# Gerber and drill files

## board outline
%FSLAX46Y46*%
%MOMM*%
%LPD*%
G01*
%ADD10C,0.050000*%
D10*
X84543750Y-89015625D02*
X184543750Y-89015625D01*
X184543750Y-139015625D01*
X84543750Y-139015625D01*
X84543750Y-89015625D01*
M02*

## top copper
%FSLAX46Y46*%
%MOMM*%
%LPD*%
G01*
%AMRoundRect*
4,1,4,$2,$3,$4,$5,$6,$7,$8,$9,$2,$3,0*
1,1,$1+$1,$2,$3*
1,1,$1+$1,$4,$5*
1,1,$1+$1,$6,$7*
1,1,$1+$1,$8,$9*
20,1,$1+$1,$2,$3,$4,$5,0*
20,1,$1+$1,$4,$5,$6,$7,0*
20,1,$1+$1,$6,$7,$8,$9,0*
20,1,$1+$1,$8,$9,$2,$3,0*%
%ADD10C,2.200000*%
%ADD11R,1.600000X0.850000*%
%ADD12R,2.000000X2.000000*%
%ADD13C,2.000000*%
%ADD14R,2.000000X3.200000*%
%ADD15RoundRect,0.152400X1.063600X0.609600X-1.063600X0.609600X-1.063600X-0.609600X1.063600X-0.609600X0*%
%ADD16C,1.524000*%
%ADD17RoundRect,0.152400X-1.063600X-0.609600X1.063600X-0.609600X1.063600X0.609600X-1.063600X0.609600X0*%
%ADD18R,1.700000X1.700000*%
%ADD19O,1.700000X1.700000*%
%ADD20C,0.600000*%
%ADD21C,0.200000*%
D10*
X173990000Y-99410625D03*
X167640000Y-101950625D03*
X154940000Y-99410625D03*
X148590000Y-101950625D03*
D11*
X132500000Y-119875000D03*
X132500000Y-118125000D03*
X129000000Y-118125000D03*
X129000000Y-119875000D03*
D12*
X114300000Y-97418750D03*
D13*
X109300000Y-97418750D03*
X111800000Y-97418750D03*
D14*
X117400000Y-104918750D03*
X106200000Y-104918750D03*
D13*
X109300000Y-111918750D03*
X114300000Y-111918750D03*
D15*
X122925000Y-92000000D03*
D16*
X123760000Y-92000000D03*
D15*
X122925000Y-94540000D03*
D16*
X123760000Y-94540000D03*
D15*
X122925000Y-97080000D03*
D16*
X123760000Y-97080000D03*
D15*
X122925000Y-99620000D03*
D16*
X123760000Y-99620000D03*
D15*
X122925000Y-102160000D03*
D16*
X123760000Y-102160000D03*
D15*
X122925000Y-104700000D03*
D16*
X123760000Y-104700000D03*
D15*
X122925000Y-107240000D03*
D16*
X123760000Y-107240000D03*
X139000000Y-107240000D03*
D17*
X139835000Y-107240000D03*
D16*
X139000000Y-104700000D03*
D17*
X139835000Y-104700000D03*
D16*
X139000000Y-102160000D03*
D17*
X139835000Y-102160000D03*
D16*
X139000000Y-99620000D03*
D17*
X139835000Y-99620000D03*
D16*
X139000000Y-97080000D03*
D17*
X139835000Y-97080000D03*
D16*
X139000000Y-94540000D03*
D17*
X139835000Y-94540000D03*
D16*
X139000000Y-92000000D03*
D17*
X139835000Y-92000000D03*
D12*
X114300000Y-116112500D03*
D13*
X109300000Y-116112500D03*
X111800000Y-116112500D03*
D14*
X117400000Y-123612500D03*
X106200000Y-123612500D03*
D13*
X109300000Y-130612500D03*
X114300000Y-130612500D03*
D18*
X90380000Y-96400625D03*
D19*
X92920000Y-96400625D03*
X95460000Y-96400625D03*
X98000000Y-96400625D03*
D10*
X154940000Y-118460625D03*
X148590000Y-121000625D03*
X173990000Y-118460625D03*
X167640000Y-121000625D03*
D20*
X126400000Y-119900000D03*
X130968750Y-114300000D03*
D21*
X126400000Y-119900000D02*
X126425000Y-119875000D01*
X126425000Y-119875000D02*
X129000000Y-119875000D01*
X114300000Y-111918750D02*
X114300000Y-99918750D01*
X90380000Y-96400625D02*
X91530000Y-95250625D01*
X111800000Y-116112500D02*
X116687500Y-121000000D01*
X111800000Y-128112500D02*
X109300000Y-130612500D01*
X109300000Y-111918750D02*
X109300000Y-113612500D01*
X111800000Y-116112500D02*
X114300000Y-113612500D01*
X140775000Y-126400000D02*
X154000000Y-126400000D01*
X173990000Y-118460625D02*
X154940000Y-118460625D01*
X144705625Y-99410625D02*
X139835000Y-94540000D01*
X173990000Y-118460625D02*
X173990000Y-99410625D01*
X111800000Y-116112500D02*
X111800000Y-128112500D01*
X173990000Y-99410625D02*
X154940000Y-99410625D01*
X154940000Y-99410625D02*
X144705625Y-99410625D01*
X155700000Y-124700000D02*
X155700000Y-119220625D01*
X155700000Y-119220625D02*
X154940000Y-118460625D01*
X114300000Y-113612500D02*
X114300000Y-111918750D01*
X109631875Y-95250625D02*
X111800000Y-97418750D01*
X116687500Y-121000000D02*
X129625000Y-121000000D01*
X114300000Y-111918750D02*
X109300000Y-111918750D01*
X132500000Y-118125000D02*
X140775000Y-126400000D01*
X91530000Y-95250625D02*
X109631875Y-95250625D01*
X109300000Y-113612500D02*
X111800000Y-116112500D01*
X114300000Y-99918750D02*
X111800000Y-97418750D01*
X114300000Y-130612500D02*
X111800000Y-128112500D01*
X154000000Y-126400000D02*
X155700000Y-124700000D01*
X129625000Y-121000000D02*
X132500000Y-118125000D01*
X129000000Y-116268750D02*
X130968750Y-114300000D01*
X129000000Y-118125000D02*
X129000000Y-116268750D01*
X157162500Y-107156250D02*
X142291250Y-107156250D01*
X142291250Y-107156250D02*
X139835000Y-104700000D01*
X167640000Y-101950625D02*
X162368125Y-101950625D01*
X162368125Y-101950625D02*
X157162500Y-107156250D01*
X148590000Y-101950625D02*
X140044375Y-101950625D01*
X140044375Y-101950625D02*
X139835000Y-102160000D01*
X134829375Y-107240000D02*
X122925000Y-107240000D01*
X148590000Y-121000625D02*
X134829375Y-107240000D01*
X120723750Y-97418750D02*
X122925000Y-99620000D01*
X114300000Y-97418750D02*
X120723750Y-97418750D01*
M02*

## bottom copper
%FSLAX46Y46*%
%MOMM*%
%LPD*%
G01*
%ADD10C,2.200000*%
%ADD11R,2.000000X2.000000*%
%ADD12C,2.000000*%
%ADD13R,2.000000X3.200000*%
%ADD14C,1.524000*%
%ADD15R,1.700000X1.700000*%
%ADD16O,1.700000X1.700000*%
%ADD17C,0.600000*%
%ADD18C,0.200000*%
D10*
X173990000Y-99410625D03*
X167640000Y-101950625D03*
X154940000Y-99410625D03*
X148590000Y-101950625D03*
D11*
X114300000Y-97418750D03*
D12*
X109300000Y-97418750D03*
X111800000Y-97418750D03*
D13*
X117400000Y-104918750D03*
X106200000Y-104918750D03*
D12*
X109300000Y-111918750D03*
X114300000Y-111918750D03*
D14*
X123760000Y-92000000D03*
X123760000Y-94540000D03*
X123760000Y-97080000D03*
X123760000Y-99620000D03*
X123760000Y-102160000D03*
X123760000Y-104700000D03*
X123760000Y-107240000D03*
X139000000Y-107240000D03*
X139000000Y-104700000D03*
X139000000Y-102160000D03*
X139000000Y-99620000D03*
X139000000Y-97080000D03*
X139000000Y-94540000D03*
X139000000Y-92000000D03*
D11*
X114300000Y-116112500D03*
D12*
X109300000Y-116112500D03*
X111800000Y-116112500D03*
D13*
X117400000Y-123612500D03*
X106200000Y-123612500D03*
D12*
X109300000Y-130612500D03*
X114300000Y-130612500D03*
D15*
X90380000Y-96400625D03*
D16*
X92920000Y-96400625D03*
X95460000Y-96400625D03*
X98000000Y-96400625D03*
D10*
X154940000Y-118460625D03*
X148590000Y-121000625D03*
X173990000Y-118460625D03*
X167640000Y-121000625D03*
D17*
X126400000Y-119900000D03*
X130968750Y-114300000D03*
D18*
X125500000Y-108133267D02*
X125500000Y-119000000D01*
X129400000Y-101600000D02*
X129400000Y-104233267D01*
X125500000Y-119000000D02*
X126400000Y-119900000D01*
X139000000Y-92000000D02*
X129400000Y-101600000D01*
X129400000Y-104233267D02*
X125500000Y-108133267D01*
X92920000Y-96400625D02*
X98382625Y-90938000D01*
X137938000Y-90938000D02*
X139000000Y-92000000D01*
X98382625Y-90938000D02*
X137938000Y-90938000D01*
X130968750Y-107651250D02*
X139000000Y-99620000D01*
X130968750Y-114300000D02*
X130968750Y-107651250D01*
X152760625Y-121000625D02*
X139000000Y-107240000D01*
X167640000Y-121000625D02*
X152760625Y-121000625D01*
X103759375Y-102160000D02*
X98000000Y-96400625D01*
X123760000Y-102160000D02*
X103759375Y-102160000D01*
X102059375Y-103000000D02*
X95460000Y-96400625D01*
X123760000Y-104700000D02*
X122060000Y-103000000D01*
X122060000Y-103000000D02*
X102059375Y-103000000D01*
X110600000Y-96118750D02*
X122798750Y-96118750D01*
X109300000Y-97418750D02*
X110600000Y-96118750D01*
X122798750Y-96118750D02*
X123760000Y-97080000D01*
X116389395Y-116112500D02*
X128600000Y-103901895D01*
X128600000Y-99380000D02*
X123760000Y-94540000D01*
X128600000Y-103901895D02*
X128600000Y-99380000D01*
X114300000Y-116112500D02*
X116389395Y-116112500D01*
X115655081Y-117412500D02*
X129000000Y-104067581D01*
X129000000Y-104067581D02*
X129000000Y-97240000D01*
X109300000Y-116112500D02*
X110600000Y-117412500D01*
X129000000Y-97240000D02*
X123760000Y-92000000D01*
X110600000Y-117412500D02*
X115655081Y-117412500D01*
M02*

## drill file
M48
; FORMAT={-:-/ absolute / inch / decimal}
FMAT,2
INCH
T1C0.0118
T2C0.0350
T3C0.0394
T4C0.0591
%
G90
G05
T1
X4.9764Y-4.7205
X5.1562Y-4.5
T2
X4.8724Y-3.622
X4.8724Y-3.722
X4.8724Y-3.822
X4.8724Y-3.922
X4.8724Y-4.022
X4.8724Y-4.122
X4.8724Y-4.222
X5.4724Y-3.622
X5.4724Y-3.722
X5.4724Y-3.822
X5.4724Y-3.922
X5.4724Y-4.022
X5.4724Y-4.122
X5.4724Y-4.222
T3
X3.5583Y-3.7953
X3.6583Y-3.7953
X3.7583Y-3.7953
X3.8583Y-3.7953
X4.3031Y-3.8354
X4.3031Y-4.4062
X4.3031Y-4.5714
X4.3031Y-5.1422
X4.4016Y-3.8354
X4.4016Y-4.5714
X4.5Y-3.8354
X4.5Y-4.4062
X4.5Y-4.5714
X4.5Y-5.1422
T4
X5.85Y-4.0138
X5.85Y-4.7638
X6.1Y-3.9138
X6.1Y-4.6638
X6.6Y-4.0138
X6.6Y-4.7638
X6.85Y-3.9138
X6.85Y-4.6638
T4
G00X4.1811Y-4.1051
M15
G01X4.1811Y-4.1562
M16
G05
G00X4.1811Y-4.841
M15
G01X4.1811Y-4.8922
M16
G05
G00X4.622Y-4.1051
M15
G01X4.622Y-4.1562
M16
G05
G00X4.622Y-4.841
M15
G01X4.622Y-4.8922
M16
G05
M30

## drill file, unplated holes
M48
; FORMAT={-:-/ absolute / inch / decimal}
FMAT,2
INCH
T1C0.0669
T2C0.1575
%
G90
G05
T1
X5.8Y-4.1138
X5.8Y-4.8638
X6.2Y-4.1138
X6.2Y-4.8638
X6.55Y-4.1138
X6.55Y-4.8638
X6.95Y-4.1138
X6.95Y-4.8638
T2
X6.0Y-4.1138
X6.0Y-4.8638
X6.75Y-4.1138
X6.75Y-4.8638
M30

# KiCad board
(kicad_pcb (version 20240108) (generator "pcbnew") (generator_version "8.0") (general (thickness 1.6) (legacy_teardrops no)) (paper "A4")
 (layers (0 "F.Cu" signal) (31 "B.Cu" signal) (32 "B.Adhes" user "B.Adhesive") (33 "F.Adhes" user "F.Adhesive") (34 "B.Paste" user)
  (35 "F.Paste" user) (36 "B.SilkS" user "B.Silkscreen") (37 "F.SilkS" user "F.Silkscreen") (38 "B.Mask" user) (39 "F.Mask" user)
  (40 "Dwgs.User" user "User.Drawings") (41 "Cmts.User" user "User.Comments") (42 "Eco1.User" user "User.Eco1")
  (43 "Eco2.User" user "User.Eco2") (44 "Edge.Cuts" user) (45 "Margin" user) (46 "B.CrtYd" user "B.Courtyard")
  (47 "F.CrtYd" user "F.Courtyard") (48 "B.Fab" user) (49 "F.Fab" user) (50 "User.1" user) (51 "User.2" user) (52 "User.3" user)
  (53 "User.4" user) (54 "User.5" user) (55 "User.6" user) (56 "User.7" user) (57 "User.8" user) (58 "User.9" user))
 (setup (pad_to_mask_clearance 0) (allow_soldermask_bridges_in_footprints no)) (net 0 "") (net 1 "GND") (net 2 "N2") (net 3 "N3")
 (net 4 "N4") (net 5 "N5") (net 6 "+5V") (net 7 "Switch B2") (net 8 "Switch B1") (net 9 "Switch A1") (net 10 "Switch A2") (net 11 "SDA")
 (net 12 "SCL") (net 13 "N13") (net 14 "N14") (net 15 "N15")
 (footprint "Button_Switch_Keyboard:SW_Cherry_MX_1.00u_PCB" (layer "F.Cu") (at 173.99 99.410625)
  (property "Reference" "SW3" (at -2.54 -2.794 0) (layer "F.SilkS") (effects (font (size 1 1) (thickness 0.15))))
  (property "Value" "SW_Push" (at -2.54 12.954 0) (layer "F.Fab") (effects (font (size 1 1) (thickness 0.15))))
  (pad "" np_thru_hole circle (at -7.62 5.08) (size 1.7 1.7) (drill 1.7) (layers "*.Cu" "*.Mask"))
  (pad "" np_thru_hole circle (at -2.54 5.08) (size 4 4) (drill 4) (layers "*.Cu" "*.Mask"))
  (pad "" np_thru_hole circle (at 2.54 5.08) (size 1.7 1.7) (drill 1.7) (layers "*.Cu" "*.Mask"))
  (pad "1" thru_hole circle (at 0 0) (size 2.2 2.2) (drill 1.5) (layers "*.Cu" "*.Mask") (remove_unused_layers no) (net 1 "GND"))
  (pad "2" thru_hole circle (at -6.35 2.54) (size 2.2 2.2) (drill 1.5) (layers "*.Cu" "*.Mask") (remove_unused_layers no) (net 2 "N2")))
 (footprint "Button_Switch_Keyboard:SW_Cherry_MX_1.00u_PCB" (layer "F.Cu") (at 154.94 99.410625)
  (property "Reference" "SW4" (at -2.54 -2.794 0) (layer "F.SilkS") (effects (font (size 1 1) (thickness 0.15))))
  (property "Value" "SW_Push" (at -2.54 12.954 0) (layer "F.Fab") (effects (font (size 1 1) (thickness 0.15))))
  (pad "" np_thru_hole circle (at -7.62 5.08) (size 1.7 1.7) (drill 1.7) (layers "*.Cu" "*.Mask"))
  (pad "" np_thru_hole circle (at -2.54 5.08) (size 4 4) (drill 4) (layers "*.Cu" "*.Mask"))
  (pad "" np_thru_hole circle (at 2.54 5.08) (size 1.7 1.7) (drill 1.7) (layers "*.Cu" "*.Mask"))
  (pad "1" thru_hole circle (at 0 0) (size 2.2 2.2) (drill 1.5) (layers "*.Cu" "*.Mask") (remove_unused_layers no) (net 1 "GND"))
  (pad "2" thru_hole circle (at -6.35 2.54) (size 2.2 2.2) (drill 1.5) (layers "*.Cu" "*.Mask") (remove_unused_layers no) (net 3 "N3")))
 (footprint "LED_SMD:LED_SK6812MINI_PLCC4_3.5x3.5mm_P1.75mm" (layer "F.Cu") (at 130.75 119 180)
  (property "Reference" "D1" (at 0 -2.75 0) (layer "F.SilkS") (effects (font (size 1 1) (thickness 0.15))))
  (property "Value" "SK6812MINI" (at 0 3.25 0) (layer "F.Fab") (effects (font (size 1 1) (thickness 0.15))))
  (pad "1" smd rect (at -1.75 -0.875 180) (size 1.6 0.85) (layers "F.Cu" "F.Paste" "F.Mask") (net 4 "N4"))
  (pad "2" smd rect (at -1.75 0.875 180) (size 1.6 0.85) (layers "F.Cu" "F.Paste" "F.Mask") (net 1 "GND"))
  (pad "3" smd rect (at 1.75 0.875 180) (size 1.6 0.85) (layers "F.Cu" "F.Paste" "F.Mask") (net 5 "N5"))
  (pad "4" smd rect (at 1.75 -0.875 180) (size 1.6 0.85) (layers "F.Cu" "F.Paste" "F.Mask") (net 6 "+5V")))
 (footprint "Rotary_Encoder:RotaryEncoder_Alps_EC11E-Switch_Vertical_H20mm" (layer "F.Cu") (at 114.3 97.41875 -90)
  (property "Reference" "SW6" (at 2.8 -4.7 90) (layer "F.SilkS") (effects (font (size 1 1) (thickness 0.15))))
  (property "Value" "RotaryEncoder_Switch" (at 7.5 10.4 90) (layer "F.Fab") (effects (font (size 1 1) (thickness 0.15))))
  (pad "A" thru_hole rect (at 0 0 270) (size 2 2) (drill 1) (layers "*.Cu" "*.Mask") (remove_unused_layers no) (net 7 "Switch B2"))
  (pad "B" thru_hole circle (at 0 5 270) (size 2 2) (drill 1) (layers "*.Cu" "*.Mask") (remove_unused_layers no) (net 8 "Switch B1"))
  (pad "C" thru_hole circle (at 0 2.5 270) (size 2 2) (drill 1) (layers "*.Cu" "*.Mask") (remove_unused_layers no) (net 1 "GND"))
  (pad "MP" thru_hole rect (at 7.5 -3.1 270) (size 3.2 2) (drill oval 2.8 1.5) (layers "*.Cu" "*.Mask") (remove_unused_layers no))
  (pad "MP" thru_hole rect (at 7.5 8.1 270) (size 3.2 2) (drill oval 2.8 1.5) (layers "*.Cu" "*.Mask") (remove_unused_layers no))
  (pad "S1" thru_hole circle (at 14.5 5 270) (size 2 2) (drill 1) (layers "*.Cu" "*.Mask") (remove_unused_layers no) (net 1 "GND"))
  (pad "S2" thru_hole circle (at 14.5 0 270) (size 2 2) (drill 1) (layers "*.Cu" "*.Mask") (remove_unused_layers no) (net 1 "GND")))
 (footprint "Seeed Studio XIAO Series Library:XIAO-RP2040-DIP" (layer "F.Cu") (at 131.38 99.62)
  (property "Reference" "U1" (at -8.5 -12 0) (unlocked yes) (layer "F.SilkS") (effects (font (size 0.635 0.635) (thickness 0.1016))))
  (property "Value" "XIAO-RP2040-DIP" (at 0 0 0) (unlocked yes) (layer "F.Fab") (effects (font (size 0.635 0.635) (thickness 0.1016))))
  (pad "1" smd roundrect (at -8.455 -7.62 180) (size 2.432 1.524) (layers "F.Cu" "F.Mask") (roundrect_rratio 0.1) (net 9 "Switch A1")
   (thermal_bridge_angle 45))
  (pad "1" thru_hole circle (at -7.62 -7.62 180) (size 1.524 1.524) (drill 0.889) (layers "*.Cu" "*.Mask") (remove_unused_layers no)
   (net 9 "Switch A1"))
  (pad "2" smd roundrect (at -8.455 -5.08 180) (size 2.432 1.524) (layers "F.Cu" "F.Mask") (roundrect_rratio 0.1) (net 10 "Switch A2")
   (thermal_bridge_angle 45))
  (pad "2" thru_hole circle (at -7.62 -5.08 180) (size 1.524 1.524) (drill 0.889) (layers "*.Cu" "*.Mask") (remove_unused_layers no)
   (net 10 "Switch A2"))
  (pad "3" smd roundrect (at -8.455 -2.54 180) (size 2.432 1.524) (layers "F.Cu" "F.Mask") (roundrect_rratio 0.1) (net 8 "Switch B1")
   (thermal_bridge_angle 45))
  (pad "3" thru_hole circle (at -7.62 -2.54 180) (size 1.524 1.524) (drill 0.889) (layers "*.Cu" "*.Mask") (remove_unused_layers no)
   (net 8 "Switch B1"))
  (pad "4" smd roundrect (at -8.455 0 180) (size 2.432 1.524) (layers "F.Cu" "F.Mask") (roundrect_rratio 0.1) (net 7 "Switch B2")
   (thermal_bridge_angle 45))
  (pad "4" thru_hole circle (at -7.62 0 180) (size 1.524 1.524) (drill 0.889) (layers "*.Cu" "*.Mask") (remove_unused_layers no)
   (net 7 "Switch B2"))
  (pad "5" smd roundrect (at -8.455 2.54 180) (size 2.432 1.524) (layers "F.Cu" "F.Mask") (roundrect_rratio 0.1) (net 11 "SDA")
   (thermal_bridge_angle 45))
  (pad "5" thru_hole circle (at -7.62 2.54 180) (size 1.524 1.524) (drill 0.889) (layers "*.Cu" "*.Mask") (remove_unused_layers no)
   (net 11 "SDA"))
  (pad "6" smd roundrect (at -8.455 5.08 180) (size 2.432 1.524) (layers "F.Cu" "F.Mask") (roundrect_rratio 0.1) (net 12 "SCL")
   (thermal_bridge_angle 45))
  (pad "6" thru_hole circle (at -7.62 5.08 180) (size 1.524 1.524) (drill 0.889) (layers "*.Cu" "*.Mask") (remove_unused_layers no)
   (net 12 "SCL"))
  (pad "7" smd roundrect (at -8.455 7.62 180) (size 2.432 1.524) (layers "F.Cu" "F.Mask") (roundrect_rratio 0.1) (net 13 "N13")
   (thermal_bridge_angle 45))
  (pad "7" thru_hole circle (at -7.62 7.62 180) (size 1.524 1.524) (drill 0.889) (layers "*.Cu" "*.Mask") (remove_unused_layers no)
   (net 13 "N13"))
  (pad "8" thru_hole circle (at 7.62 7.62) (size 1.524 1.524) (drill 0.889) (layers "*.Cu" "*.Mask") (remove_unused_layers no)
   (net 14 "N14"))
  (pad "8" smd roundrect (at 8.455 7.62) (size 2.432 1.524) (layers "F.Cu" "F.Mask") (roundrect_rratio 0.1) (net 14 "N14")
   (thermal_bridge_angle 45))
  (pad "9" thru_hole circle (at 7.62 5.08) (size 1.524 1.524) (drill 0.889) (layers "*.Cu" "*.Mask") (remove_unused_layers no) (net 2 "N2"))
  (pad "9" smd roundrect (at 8.455 5.08) (size 2.432 1.524) (layers "F.Cu" "F.Mask") (roundrect_rratio 0.1) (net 2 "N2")
   (thermal_bridge_angle 45))
  (pad "10" thru_hole circle (at 7.62 2.54) (size 1.524 1.524) (drill 0.889) (layers "*.Cu" "*.Mask") (remove_unused_layers no) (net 3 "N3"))
  (pad "10" smd roundrect (at 8.455 2.54) (size 2.432 1.524) (layers "F.Cu" "F.Mask") (roundrect_rratio 0.1) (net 3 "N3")
   (thermal_bridge_angle 45))
  (pad "11" thru_hole circle (at 7.62 0) (size 1.524 1.524) (drill 0.889) (layers "*.Cu" "*.Mask") (remove_unused_layers no) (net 5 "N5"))
  (pad "11" smd roundrect (at 8.455 0) (size 2.432 1.524) (layers "F.Cu" "F.Mask") (roundrect_rratio 0.1) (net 5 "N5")
   (thermal_bridge_angle 45))
  (pad "12" thru_hole circle (at 7.62 -2.54) (size 1.524 1.524) (drill 0.889) (layers "*.Cu" "*.Mask") (remove_unused_layers no)
   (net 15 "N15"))
  (pad "12" smd roundrect (at 8.455 -2.54) (size 2.432 1.524) (layers "F.Cu" "F.Mask") (roundrect_rratio 0.1) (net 15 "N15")
   (thermal_bridge_angle 45))
  (pad "13" thru_hole circle (at 7.62 -5.08) (size 1.524 1.524) (drill 0.889) (layers "*.Cu" "*.Mask") (remove_unused_layers no)
   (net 1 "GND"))
  (pad "13" smd roundrect (at 8.455 -5.08) (size 2.432 1.524) (layers "F.Cu" "F.Mask") (roundrect_rratio 0.1) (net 1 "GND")
   (thermal_bridge_angle 45))
  (pad "14" thru_hole circle (at 7.62 -7.62) (size 1.524 1.524) (drill 0.889) (layers "*.Cu" "*.Mask") (remove_unused_layers no)
   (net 6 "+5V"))
  (pad "14" smd roundrect (at 8.455 -7.62) (size 2.432 1.524) (layers "F.Cu" "F.Mask") (roundrect_rratio 0.1) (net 6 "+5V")
   (thermal_bridge_angle 45)))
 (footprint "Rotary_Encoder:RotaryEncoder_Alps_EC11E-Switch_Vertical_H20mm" (layer "F.Cu") (at 114.3 116.1125 -90)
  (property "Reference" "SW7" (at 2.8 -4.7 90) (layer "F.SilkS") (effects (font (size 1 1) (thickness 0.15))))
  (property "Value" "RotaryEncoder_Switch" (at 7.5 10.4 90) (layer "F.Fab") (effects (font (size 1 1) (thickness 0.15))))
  (pad "A" thru_hole rect (at 0 0 270) (size 2 2) (drill 1) (layers "*.Cu" "*.Mask") (remove_unused_layers no) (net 10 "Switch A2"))
  (pad "B" thru_hole circle (at 0 5 270) (size 2 2) (drill 1) (layers "*.Cu" "*.Mask") (remove_unused_layers no) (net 9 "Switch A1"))
  (pad "C" thru_hole circle (at 0 2.5 270) (size 2 2) (drill 1) (layers "*.Cu" "*.Mask") (remove_unused_layers no) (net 1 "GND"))
  (pad "MP" thru_hole rect (at 7.5 -3.1 270) (size 3.2 2) (drill oval 2.8 1.5) (layers "*.Cu" "*.Mask") (remove_unused_layers no))
  (pad "MP" thru_hole rect (at 7.5 8.1 270) (size 3.2 2) (drill oval 2.8 1.5) (layers "*.Cu" "*.Mask") (remove_unused_layers no))
  (pad "S1" thru_hole circle (at 14.5 5 270) (size 2 2) (drill 1) (layers "*.Cu" "*.Mask") (remove_unused_layers no) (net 1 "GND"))
  (pad "S2" thru_hole circle (at 14.5 0 270) (size 2 2) (drill 1) (layers "*.Cu" "*.Mask") (remove_unused_layers no) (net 1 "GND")))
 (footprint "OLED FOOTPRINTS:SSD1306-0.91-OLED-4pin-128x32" (layer "F.Cu") (at 88.19 132.900625 90)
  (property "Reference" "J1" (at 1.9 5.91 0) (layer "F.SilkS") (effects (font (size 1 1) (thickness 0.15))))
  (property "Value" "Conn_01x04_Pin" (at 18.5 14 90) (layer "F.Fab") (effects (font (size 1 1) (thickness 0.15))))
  (pad "1" thru_hole rect (at 36.5 2.19 90) (size 1.7 1.7) (drill 1) (layers "*.Cu" "*.Mask") (remove_unused_layers no) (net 1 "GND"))
  (pad "2" thru_hole oval (at 36.5 4.73 90) (size 1.7 1.7) (drill 1) (layers "*.Cu" "*.Mask") (remove_unused_layers no) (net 6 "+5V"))
  (pad "3" thru_hole oval (at 36.5 7.27 90) (size 1.7 1.7) (drill 1) (layers "*.Cu" "*.Mask") (remove_unused_layers no) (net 12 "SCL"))
  (pad "4" thru_hole oval (at 36.5 9.81 90) (size 1.7 1.7) (drill 1) (layers "*.Cu" "*.Mask") (remove_unused_layers no) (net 11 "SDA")))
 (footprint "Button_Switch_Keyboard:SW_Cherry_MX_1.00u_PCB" (layer "F.Cu") (at 154.94 118.460625)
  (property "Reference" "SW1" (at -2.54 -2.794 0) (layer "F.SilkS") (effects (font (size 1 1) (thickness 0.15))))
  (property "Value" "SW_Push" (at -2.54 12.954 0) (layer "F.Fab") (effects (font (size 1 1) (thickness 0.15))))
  (pad "" np_thru_hole circle (at -7.62 5.08) (size 1.7 1.7) (drill 1.7) (layers "*.Cu" "*.Mask"))
  (pad "" np_thru_hole circle (at -2.54 5.08) (size 4 4) (drill 4) (layers "*.Cu" "*.Mask"))
  (pad "" np_thru_hole circle (at 2.54 5.08) (size 1.7 1.7) (drill 1.7) (layers "*.Cu" "*.Mask"))
  (pad "1" thru_hole circle (at 0 0) (size 2.2 2.2) (drill 1.5) (layers "*.Cu" "*.Mask") (remove_unused_layers no) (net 1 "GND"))
  (pad "2" thru_hole circle (at -6.35 2.54) (size 2.2 2.2) (drill 1.5) (layers "*.Cu" "*.Mask") (remove_unused_layers no) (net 13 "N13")))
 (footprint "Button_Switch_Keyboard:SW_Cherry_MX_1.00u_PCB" (layer "F.Cu") (at 173.99 118.460625)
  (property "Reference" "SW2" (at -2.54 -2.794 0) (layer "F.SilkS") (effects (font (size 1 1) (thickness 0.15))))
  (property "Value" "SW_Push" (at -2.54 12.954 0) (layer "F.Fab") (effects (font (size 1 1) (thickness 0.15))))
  (pad "" np_thru_hole circle (at -7.62 5.08) (size 1.7 1.7) (drill 1.7) (layers "*.Cu" "*.Mask"))
  (pad "" np_thru_hole circle (at -2.54 5.08) (size 4 4) (drill 4) (layers "*.Cu" "*.Mask"))
  (pad "" np_thru_hole circle (at 2.54 5.08) (size 1.7 1.7) (drill 1.7) (layers "*.Cu" "*.Mask"))
  (pad "1" thru_hole circle (at 0 0) (size 2.2 2.2) (drill 1.5) (layers "*.Cu" "*.Mask") (remove_unused_layers no) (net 1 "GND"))
  (pad "2" thru_hole circle (at -6.35 2.54) (size 2.2 2.2) (drill 1.5) (layers "*.Cu" "*.Mask") (remove_unused_layers no) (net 14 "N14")))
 (gr_rect (start 84.54375 89.015625) (end 184.54375 139.015625) (stroke (width 0.05) (type default)) (fill none) (layer "Edge.Cuts"))
 (segment (start 126.4 119.9) (end 126.425 119.875) (width 0.2) (layer "F.Cu") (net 6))
 (segment (start 126.425 119.875) (end 129 119.875) (width 0.2) (layer "F.Cu") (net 6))
 (via (at 126.4 119.9) (size 0.6) (drill 0.3) (layers "F.Cu" "B.Cu") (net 6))
 (segment (start 125.5 108.133267) (end 125.5 119) (width 0.2) (layer "B.Cu") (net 6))
 (segment (start 129.4 101.6) (end 129.4 104.233267) (width 0.2) (layer "B.Cu") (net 6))
 (segment (start 125.5 119) (end 126.4 119.9) (width 0.2) (layer "B.Cu") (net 6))
 (segment (start 139 92) (end 129.4 101.6) (width 0.2) (layer "B.Cu") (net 6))
 (segment (start 129.4 104.233267) (end 125.5 108.133267) (width 0.2) (layer "B.Cu") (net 6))
 (segment (start 92.92 96.400625) (end 98.382625 90.938) (width 0.2) (layer "B.Cu") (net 6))
 (segment (start 137.938 90.938) (end 139 92) (width 0.2) (layer "B.Cu") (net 6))
 (segment (start 98.382625 90.938) (end 137.938 90.938) (width 0.2) (layer "B.Cu") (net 6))
 (segment (start 114.3 111.91875) (end 114.3 99.91875) (width 0.2) (layer "F.Cu") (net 1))
 (segment (start 90.38 96.400625) (end 91.53 95.250625) (width 0.2) (layer "F.Cu") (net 1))
 (segment (start 111.8 116.1125) (end 116.6875 121) (width 0.2) (layer "F.Cu") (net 1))
 (segment (start 111.8 128.1125) (end 109.3 130.6125) (width 0.2) (layer "F.Cu") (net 1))
 (segment (start 109.3 111.91875) (end 109.3 113.6125) (width 0.2) (layer "F.Cu") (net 1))
 (segment (start 111.8 116.1125) (end 114.3 113.6125) (width 0.2) (layer "F.Cu") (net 1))
 (segment (start 140.775 126.4) (end 154 126.4) (width 0.2) (layer "F.Cu") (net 1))
 (segment (start 173.99 118.460625) (end 154.94 118.460625) (width 0.2) (layer "F.Cu") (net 1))
 (segment (start 144.705625 99.410625) (end 139.835 94.54) (width 0.2) (layer "F.Cu") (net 1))
 (segment (start 173.99 118.460625) (end 173.99 99.410625) (width 0.2) (layer "F.Cu") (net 1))
 (segment (start 111.8 116.1125) (end 111.8 128.1125) (width 0.2) (layer "F.Cu") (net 1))
 (segment (start 173.99 99.410625) (end 154.94 99.410625) (width 0.2) (layer "F.Cu") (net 1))
 (segment (start 154.94 99.410625) (end 144.705625 99.410625) (width 0.2) (layer "F.Cu") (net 1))
 (segment (start 155.7 124.7) (end 155.7 119.220625) (width 0.2) (layer "F.Cu") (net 1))
 (segment (start 155.7 119.220625) (end 154.94 118.460625) (width 0.2) (layer "F.Cu") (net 1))
 (segment (start 114.3 113.6125) (end 114.3 111.91875) (width 0.2) (layer "F.Cu") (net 1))
 (segment (start 109.631875 95.250625) (end 111.8 97.41875) (width 0.2) (layer "F.Cu") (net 1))
 (segment (start 116.6875 121) (end 129.625 121) (width 0.2) (layer "F.Cu") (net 1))
 (segment (start 114.3 111.91875) (end 109.3 111.91875) (width 0.2) (layer "F.Cu") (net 1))
 (segment (start 132.5 118.125) (end 140.775 126.4) (width 0.2) (layer "F.Cu") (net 1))
 (segment (start 91.53 95.250625) (end 109.631875 95.250625) (width 0.2) (layer "F.Cu") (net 1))
 (segment (start 109.3 113.6125) (end 111.8 116.1125) (width 0.2) (layer "F.Cu") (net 1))
 (segment (start 114.3 99.91875) (end 111.8 97.41875) (width 0.2) (layer "F.Cu") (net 1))
 (segment (start 114.3 130.6125) (end 111.8 128.1125) (width 0.2) (layer "F.Cu") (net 1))
 (segment (start 154 126.4) (end 155.7 124.7) (width 0.2) (layer "F.Cu") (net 1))
 (segment (start 129.625 121) (end 132.5 118.125) (width 0.2) (layer "F.Cu") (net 1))
 (segment (start 129 116.26875) (end 130.96875 114.3) (width 0.2) (layer "F.Cu") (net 5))
 (segment (start 129 118.125) (end 129 116.26875) (width 0.2) (layer "F.Cu") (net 5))
 (via (at 130.96875 114.3) (size 0.6) (drill 0.3) (layers "F.Cu" "B.Cu") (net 5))
 (segment (start 130.96875 107.65125) (end 139 99.62) (width 0.2) (layer "B.Cu") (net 5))
 (segment (start 130.96875 114.3) (end 130.96875 107.65125) (width 0.2) (layer "B.Cu") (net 5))
 (segment (start 152.760625 121.000625) (end 139 107.24) (width 0.2) (layer "B.Cu") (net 14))
 (segment (start 167.64 121.000625) (end 152.760625 121.000625) (width 0.2) (layer "B.Cu") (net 14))
 (segment (start 157.1625 107.15625) (end 142.29125 107.15625) (width 0.2) (layer "F.Cu") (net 2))
 (segment (start 142.29125 107.15625) (end 139.835 104.7) (width 0.2) (layer "F.Cu") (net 2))
 (segment (start 167.64 101.950625) (end 162.368125 101.950625) (width 0.2) (layer "F.Cu") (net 2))
 (segment (start 162.368125 101.950625) (end 157.1625 107.15625) (width 0.2) (layer "F.Cu") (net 2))
 (segment (start 148.59 101.950625) (end 140.044375 101.950625) (width 0.2) (layer "F.Cu") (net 3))
 (segment (start 140.044375 101.950625) (end 139.835 102.16) (width 0.2) (layer "F.Cu") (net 3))
 (segment (start 103.759375 102.16) (end 98 96.400625) (width 0.2) (layer "B.Cu") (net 11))
 (segment (start 123.76 102.16) (end 103.759375 102.16) (width 0.2) (layer "B.Cu") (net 11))
 (segment (start 102.059375 103) (end 95.46 96.400625) (width 0.2) (layer "B.Cu") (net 12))
 (segment (start 123.76 104.7) (end 122.06 103) (width 0.2) (layer "B.Cu") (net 12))
 (segment (start 122.06 103) (end 102.059375 103) (width 0.2) (layer "B.Cu") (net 12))
 (segment (start 134.829375 107.24) (end 122.925 107.24) (width 0.2) (layer "F.Cu") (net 13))
 (segment (start 148.59 121.000625) (end 134.829375 107.24) (width 0.2) (layer "F.Cu") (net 13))
 (segment (start 120.72375 97.41875) (end 122.925 99.62) (width 0.2) (layer "F.Cu") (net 7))
 (segment (start 114.3 97.41875) (end 120.72375 97.41875) (width 0.2) (layer "F.Cu") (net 7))
 (segment (start 110.6 96.11875) (end 122.79875 96.11875) (width 0.2) (layer "B.Cu") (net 8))
 (segment (start 109.3 97.41875) (end 110.6 96.11875) (width 0.2) (layer "B.Cu") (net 8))
 (segment (start 122.79875 96.11875) (end 123.76 97.08) (width 0.2) (layer "B.Cu") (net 8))
 (segment (start 116.389395 116.1125) (end 128.6 103.901895) (width 0.2) (layer "B.Cu") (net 10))
 (segment (start 128.6 99.38) (end 123.76 94.54) (width 0.2) (layer "B.Cu") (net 10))
 (segment (start 128.6 103.901895) (end 128.6 99.38) (width 0.2) (layer "B.Cu") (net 10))
 (segment (start 114.3 116.1125) (end 116.389395 116.1125) (width 0.2) (layer "B.Cu") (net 10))
 (segment (start 115.655081 117.4125) (end 129 104.067581) (width 0.2) (layer "B.Cu") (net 9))
 (segment (start 129 104.067581) (end 129 97.24) (width 0.2) (layer "B.Cu") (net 9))
 (segment (start 109.3 116.1125) (end 110.6 117.4125) (width 0.2) (layer "B.Cu") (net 9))
 (segment (start 129 97.24) (end 123.76 92) (width 0.2) (layer "B.Cu") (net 9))
 (segment (start 110.6 117.4125) (end 115.655081 117.4125) (width 0.2) (layer "B.Cu") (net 9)))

